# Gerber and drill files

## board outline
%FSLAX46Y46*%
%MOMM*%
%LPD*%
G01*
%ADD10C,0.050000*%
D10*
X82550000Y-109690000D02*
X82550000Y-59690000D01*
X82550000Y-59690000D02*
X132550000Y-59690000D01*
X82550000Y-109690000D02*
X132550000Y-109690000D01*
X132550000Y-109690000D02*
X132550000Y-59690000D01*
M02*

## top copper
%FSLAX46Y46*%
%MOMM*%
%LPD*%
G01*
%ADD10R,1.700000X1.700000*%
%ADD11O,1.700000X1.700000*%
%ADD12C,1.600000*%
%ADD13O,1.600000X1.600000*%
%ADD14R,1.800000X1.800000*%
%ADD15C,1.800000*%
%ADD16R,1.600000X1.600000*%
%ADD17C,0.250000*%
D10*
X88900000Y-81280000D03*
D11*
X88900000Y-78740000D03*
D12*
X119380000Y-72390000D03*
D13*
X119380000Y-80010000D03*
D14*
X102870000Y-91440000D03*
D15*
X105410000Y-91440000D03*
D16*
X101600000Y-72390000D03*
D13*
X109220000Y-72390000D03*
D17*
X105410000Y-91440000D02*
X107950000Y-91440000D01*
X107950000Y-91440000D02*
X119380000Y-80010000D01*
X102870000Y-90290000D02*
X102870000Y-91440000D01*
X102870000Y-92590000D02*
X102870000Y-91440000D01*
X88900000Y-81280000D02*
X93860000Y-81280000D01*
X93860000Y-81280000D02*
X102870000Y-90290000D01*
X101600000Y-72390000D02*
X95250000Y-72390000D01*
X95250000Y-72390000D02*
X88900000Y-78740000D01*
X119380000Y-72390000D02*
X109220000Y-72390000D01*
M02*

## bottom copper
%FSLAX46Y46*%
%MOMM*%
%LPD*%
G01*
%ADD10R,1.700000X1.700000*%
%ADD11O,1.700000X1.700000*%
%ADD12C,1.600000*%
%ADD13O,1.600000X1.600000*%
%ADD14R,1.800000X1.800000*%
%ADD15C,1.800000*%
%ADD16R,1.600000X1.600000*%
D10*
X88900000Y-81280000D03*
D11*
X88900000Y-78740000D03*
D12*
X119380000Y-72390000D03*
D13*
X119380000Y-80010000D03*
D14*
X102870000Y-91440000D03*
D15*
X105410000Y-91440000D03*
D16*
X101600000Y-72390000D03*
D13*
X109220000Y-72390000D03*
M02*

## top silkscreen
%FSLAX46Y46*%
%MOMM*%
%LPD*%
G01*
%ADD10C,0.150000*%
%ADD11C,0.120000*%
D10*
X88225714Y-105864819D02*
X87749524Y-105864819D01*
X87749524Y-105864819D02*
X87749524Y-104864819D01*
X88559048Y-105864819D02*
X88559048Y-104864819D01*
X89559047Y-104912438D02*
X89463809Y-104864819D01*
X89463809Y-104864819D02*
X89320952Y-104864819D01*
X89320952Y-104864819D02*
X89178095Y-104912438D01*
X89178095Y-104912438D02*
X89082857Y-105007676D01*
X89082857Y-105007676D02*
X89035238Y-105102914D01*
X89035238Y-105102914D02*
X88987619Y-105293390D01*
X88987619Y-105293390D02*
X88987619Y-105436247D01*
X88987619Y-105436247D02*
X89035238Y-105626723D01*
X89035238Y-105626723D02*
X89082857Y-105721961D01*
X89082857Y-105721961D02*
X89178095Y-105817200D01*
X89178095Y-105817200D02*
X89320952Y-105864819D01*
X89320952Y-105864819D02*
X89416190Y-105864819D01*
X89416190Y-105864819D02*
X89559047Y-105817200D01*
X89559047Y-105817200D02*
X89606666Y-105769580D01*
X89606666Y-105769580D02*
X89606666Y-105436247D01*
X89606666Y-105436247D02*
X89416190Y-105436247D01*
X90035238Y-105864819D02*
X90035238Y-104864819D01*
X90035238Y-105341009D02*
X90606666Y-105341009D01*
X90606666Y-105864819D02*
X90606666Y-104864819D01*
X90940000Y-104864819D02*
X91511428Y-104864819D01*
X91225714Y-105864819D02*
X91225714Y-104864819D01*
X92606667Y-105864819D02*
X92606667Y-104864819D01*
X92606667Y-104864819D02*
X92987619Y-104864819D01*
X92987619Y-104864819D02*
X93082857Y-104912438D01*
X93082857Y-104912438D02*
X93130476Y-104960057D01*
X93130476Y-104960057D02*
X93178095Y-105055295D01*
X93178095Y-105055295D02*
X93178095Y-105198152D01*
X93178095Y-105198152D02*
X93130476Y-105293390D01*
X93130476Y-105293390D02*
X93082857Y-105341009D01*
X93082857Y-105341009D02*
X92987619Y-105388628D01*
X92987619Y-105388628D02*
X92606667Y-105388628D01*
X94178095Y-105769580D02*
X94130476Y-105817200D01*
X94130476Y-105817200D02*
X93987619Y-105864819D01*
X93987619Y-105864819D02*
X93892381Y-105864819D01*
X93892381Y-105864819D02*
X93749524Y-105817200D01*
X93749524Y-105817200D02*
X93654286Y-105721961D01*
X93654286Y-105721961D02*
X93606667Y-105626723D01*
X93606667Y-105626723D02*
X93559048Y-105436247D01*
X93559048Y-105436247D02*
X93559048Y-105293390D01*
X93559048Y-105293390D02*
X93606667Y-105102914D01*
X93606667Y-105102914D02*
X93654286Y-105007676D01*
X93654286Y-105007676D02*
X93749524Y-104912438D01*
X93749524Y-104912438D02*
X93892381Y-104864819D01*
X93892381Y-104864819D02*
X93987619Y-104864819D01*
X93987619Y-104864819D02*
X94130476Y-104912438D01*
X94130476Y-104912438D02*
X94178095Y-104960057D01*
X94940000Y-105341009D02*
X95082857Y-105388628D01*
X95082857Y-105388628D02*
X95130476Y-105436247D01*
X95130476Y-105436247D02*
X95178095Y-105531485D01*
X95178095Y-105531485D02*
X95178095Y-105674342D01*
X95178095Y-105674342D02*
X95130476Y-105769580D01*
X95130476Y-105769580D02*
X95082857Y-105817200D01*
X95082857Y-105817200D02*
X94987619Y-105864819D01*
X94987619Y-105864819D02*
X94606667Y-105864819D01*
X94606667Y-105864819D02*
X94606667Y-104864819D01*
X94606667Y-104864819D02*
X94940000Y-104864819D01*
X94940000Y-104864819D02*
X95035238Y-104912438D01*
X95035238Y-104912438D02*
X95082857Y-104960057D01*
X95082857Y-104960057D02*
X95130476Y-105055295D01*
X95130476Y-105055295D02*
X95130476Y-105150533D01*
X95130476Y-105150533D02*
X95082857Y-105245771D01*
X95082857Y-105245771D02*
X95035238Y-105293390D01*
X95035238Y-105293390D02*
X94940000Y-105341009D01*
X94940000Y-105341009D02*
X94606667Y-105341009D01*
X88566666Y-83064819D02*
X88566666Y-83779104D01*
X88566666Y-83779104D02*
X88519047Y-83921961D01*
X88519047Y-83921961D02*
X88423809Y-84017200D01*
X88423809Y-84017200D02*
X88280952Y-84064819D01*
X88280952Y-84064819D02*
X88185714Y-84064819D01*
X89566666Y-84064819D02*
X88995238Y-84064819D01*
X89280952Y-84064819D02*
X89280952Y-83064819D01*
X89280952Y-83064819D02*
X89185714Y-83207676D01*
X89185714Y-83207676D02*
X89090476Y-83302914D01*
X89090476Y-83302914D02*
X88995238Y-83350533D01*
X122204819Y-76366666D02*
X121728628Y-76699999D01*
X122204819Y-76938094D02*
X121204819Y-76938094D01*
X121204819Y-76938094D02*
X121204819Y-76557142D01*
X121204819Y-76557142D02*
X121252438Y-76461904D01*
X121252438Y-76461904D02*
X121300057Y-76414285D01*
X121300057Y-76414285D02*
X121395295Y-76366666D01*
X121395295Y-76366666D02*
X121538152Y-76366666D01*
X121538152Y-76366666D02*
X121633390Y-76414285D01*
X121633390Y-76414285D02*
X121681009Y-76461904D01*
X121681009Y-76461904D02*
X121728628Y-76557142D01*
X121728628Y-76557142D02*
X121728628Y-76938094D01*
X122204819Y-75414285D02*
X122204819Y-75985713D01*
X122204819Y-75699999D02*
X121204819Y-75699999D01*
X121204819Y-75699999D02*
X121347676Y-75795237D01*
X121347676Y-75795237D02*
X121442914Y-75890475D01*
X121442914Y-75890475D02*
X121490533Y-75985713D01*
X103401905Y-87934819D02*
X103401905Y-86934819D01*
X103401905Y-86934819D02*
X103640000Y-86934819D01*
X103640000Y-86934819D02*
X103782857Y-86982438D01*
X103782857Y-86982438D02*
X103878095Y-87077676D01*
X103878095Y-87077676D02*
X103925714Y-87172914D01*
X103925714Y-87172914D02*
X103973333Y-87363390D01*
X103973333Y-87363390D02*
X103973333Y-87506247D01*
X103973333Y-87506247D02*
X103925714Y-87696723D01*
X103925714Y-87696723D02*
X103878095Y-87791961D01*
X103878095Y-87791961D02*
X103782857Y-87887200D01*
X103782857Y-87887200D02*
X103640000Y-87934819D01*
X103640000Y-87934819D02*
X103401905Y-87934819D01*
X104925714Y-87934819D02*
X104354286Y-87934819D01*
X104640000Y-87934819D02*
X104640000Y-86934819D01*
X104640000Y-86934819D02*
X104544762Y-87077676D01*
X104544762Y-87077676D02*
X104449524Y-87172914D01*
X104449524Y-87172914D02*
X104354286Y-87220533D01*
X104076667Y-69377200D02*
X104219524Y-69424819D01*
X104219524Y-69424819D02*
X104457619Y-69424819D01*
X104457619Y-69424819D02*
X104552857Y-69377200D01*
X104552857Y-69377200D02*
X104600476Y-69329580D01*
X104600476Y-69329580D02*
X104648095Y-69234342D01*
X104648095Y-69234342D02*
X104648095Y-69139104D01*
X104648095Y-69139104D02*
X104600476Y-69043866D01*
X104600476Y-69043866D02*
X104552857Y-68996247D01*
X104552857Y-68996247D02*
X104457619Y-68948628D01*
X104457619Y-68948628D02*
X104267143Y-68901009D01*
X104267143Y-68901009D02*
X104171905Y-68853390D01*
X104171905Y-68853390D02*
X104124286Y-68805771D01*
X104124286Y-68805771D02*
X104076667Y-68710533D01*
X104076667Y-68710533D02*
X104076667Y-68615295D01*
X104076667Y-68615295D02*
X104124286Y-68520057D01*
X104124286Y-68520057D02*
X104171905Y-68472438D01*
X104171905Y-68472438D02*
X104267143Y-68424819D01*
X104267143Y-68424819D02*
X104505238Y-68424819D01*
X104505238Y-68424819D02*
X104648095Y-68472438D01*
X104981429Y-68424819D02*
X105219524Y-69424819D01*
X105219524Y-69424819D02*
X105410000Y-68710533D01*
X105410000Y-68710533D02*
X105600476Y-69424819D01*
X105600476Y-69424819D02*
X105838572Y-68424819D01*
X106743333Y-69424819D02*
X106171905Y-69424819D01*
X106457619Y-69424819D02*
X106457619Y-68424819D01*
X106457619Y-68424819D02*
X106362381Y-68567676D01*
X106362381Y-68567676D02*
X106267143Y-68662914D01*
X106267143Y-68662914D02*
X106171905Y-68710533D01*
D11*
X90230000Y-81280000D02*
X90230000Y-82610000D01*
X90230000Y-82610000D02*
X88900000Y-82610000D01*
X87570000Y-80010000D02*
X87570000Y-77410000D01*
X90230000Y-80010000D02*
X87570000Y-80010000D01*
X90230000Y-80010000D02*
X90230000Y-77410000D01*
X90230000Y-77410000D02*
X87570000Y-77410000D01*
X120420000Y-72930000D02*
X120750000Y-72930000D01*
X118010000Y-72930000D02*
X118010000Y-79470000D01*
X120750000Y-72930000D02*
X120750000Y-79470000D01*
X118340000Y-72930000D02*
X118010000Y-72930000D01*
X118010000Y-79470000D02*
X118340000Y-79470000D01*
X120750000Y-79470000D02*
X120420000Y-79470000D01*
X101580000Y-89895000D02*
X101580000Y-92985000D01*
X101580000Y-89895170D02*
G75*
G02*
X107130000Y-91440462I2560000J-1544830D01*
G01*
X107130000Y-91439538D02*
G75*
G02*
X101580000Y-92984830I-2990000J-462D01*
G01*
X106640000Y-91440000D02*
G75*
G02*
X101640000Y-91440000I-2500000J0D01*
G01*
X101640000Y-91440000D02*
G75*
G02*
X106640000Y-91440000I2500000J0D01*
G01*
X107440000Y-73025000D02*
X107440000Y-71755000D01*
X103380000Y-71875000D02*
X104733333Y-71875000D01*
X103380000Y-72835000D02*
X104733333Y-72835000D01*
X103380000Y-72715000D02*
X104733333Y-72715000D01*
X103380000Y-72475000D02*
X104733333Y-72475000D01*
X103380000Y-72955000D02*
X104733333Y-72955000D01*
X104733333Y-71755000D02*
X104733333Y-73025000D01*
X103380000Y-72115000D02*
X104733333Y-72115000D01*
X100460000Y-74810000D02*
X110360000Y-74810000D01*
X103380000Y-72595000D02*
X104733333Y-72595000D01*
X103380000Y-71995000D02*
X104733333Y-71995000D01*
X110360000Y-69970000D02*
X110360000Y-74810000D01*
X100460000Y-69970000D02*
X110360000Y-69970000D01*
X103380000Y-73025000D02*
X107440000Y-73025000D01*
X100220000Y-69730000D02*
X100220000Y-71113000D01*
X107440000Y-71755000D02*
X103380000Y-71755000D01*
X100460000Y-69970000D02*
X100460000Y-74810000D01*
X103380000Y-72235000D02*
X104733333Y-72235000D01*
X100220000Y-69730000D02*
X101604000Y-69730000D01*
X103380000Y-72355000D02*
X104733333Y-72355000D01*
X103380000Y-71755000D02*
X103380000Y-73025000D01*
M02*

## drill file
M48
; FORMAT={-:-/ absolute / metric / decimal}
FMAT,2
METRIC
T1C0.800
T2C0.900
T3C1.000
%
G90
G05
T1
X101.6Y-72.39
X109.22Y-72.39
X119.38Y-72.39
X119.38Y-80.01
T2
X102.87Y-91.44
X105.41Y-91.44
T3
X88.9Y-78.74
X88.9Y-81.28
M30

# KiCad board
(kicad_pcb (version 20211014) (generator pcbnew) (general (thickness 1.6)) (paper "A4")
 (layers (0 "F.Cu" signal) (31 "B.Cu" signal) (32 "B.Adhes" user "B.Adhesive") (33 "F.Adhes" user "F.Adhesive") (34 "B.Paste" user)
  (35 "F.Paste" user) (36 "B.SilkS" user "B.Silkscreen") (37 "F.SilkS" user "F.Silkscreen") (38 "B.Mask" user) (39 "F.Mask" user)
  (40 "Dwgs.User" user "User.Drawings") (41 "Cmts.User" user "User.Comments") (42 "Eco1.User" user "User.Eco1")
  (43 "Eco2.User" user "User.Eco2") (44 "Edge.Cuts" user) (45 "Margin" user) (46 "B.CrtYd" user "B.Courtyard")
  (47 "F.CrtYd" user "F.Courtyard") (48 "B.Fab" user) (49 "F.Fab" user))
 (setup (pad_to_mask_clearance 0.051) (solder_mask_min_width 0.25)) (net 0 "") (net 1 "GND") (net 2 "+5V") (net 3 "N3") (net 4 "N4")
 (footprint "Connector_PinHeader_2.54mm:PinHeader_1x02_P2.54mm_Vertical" (layer "F.Cu") (at 88.9 81.28 180)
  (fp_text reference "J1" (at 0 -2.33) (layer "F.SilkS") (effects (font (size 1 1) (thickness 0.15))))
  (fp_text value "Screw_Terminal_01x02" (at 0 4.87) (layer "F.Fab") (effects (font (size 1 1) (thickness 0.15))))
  (fp_line (start -1.33 0) (end -1.33 -1.33) (layer "F.SilkS") (width 0.12))
  (fp_line (start -1.33 -1.33) (end 0 -1.33) (layer "F.SilkS") (width 0.12))
  (fp_line (start 1.33 1.27) (end 1.33 3.87) (layer "F.SilkS") (width 0.12))
  (fp_line (start -1.33 1.27) (end 1.33 1.27) (layer "F.SilkS") (width 0.12))
  (fp_line (start -1.33 1.27) (end -1.33 3.87) (layer "F.SilkS") (width 0.12))
  (fp_line (start -1.33 3.87) (end 1.33 3.87) (layer "F.SilkS") (width 0.12))
  (pad "1" thru_hole rect locked (at 0 0 180) (size 1.7 1.7) (drill 1) (layers *.Cu *.Mask) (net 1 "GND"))
  (pad "2" thru_hole oval locked (at 0 2.54 180) (size 1.7 1.7) (drill 1) (layers *.Cu *.Mask) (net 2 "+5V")))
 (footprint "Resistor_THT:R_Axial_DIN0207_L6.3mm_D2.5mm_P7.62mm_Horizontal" (layer "F.Cu") (at 119.38 72.39 -90)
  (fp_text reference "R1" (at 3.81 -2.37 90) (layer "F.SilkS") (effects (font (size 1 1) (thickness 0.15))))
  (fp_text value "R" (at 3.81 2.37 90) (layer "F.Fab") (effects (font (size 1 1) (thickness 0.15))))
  (fp_line (start 0.54 -1.04) (end 0.54 -1.37) (layer "F.SilkS") (width 0.12))
  (fp_line (start 0.54 1.37) (end 7.08 1.37) (layer "F.SilkS") (width 0.12))
  (fp_line (start 0.54 -1.37) (end 7.08 -1.37) (layer "F.SilkS") (width 0.12))
  (fp_line (start 0.54 1.04) (end 0.54 1.37) (layer "F.SilkS") (width 0.12))
  (fp_line (start 7.08 1.37) (end 7.08 1.04) (layer "F.SilkS") (width 0.12))
  (fp_line (start 7.08 -1.37) (end 7.08 -1.04) (layer "F.SilkS") (width 0.12))
  (pad "1" thru_hole circle locked (at 0 0 270) (size 1.6 1.6) (drill 0.8) (layers *.Cu *.Mask) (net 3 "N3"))
  (pad "2" thru_hole oval locked (at 7.62 0 270) (size 1.6 1.6) (drill 0.8) (layers *.Cu *.Mask) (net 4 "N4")))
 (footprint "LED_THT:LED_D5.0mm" (layer "F.Cu") (at 102.87 91.44)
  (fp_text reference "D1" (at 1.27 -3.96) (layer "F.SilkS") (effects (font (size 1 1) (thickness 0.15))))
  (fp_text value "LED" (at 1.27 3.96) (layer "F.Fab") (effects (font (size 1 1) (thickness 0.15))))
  (fp_line (start -1.29 -1.545) (end -1.29 1.545) (layer "F.SilkS") (width 0.12))
  (fp_arc (start -1.29 -1.54483) (mid 2.072002 -2.880433) (end 4.26 0.000462) (layer "F.SilkS") (width 0.12))
  (fp_arc (start 4.26 -0.000462) (mid 2.072002 2.880433) (end -1.29 1.54483) (layer "F.SilkS") (width 0.12))
  (fp_circle (center 1.27 0) (end 3.77 0) (layer "F.SilkS") (width 0.12) (fill none))
  (pad "1" thru_hole rect locked (at 0 0) (size 1.8 1.8) (drill 0.9) (layers *.Cu *.Mask) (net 1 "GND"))
  (pad "2" thru_hole circle locked (at 2.54 0) (size 1.8 1.8) (drill 0.9) (layers *.Cu *.Mask) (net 4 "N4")))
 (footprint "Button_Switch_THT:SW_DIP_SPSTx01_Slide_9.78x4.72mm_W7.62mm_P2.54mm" (layer "F.Cu") (at 101.6 72.39)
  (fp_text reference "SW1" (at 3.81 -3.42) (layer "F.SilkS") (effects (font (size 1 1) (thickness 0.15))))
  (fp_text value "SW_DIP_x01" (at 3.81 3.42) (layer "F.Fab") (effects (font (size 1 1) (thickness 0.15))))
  (fp_line (start 5.84 0.635) (end 5.84 -0.635) (layer "F.SilkS") (width 0.12))
  (fp_line (start 1.78 -0.515) (end 3.133333 -0.515) (layer "F.SilkS") (width 0.12))
  (fp_line (start 1.78 0.445) (end 3.133333 0.445) (layer "F.SilkS") (width 0.12))
  (fp_line (start 1.78 0.325) (end 3.133333 0.325) (layer "F.SilkS") (width 0.12))
  (fp_line (start 1.78 0.085) (end 3.133333 0.085) (layer "F.SilkS") (width 0.12))
  (fp_line (start 1.78 0.565) (end 3.133333 0.565) (layer "F.SilkS") (width 0.12))
  (fp_line (start 3.133333 -0.635) (end 3.133333 0.635) (layer "F.SilkS") (width 0.12))
  (fp_line (start 1.78 -0.275) (end 3.133333 -0.275) (layer "F.SilkS") (width 0.12))
  (fp_line (start -1.14 2.42) (end 8.76 2.42) (layer "F.SilkS") (width 0.12))
  (fp_line (start 1.78 0.205) (end 3.133333 0.205) (layer "F.SilkS") (width 0.12))
  (fp_line (start 1.78 -0.395) (end 3.133333 -0.395) (layer "F.SilkS") (width 0.12))
  (fp_line (start 8.76 -2.42) (end 8.76 2.42) (layer "F.SilkS") (width 0.12))
  (fp_line (start -1.14 -2.42) (end 8.76 -2.42) (layer "F.SilkS") (width 0.12))
  (fp_line (start 1.78 0.635) (end 5.84 0.635) (layer "F.SilkS") (width 0.12))
  (fp_line (start -1.38 -2.66) (end -1.38 -1.277) (layer "F.SilkS") (width 0.12))
  (fp_line (start 5.84 -0.635) (end 1.78 -0.635) (layer "F.SilkS") (width 0.12))
  (fp_line (start -1.14 -2.42) (end -1.14 2.42) (layer "F.SilkS") (width 0.12))
  (fp_line (start 1.78 -0.155) (end 3.133333 -0.155) (layer "F.SilkS") (width 0.12))
  (fp_line (start -1.38 -2.66) (end 0.004 -2.66) (layer "F.SilkS") (width 0.12))
  (fp_line (start 1.78 -0.035) (end 3.133333 -0.035) (layer "F.SilkS") (width 0.12))
  (fp_line (start 1.78 -0.635) (end 1.78 0.635) (layer "F.SilkS") (width 0.12))
  (pad "1" thru_hole rect locked (at 0 0) (size 1.6 1.6) (drill 0.8) (layers *.Cu *.Mask) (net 2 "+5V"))
  (pad "2" thru_hole oval locked (at 7.62 0) (size 1.6 1.6) (drill 0.8) (layers *.Cu *.Mask) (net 3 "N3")))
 (gr_line (start 82.55 109.69) (end 82.55 59.69) (layer "Edge.Cuts") (width 0.05))
 (gr_line (start 82.55 59.69) (end 132.55 59.69) (layer "Edge.Cuts") (width 0.05))
 (gr_line (start 82.55 109.69) (end 132.55 109.69) (layer "Edge.Cuts") (width 0.05))
 (gr_line (start 132.55 109.69) (end 132.55 59.69) (layer "Edge.Cuts") (width 0.05))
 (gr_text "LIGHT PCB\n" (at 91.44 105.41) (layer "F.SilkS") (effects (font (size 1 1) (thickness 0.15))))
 (segment (start 105.41 91.44) (end 107.95 91.44) (width 0.25) (layer "F.Cu") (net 4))
 (segment (start 107.95 91.44) (end 119.38 80.01) (width 0.25) (layer "F.Cu") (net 4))
 (segment (start 102.87 90.29) (end 102.87 91.44) (width 0.25) (layer "F.Cu") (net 1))
 (segment (start 102.87 92.59) (end 102.87 91.44) (width 0.25) (layer "F.Cu") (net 1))
 (segment (start 88.9 81.28) (end 93.86 81.28) (width 0.25) (layer "F.Cu") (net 1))
 (segment (start 93.86 81.28) (end 102.87 90.29) (width 0.25) (layer "F.Cu") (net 1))
 (segment (start 101.6 72.39) (end 95.25 72.39) (width 0.25) (layer "F.Cu") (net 2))
 (segment (start 95.25 72.39) (end 88.9 78.74) (width 0.25) (layer "F.Cu") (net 2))
 (segment (start 119.38 72.39) (end 109.22 72.39) (width 0.25) (layer "F.Cu") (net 3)))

